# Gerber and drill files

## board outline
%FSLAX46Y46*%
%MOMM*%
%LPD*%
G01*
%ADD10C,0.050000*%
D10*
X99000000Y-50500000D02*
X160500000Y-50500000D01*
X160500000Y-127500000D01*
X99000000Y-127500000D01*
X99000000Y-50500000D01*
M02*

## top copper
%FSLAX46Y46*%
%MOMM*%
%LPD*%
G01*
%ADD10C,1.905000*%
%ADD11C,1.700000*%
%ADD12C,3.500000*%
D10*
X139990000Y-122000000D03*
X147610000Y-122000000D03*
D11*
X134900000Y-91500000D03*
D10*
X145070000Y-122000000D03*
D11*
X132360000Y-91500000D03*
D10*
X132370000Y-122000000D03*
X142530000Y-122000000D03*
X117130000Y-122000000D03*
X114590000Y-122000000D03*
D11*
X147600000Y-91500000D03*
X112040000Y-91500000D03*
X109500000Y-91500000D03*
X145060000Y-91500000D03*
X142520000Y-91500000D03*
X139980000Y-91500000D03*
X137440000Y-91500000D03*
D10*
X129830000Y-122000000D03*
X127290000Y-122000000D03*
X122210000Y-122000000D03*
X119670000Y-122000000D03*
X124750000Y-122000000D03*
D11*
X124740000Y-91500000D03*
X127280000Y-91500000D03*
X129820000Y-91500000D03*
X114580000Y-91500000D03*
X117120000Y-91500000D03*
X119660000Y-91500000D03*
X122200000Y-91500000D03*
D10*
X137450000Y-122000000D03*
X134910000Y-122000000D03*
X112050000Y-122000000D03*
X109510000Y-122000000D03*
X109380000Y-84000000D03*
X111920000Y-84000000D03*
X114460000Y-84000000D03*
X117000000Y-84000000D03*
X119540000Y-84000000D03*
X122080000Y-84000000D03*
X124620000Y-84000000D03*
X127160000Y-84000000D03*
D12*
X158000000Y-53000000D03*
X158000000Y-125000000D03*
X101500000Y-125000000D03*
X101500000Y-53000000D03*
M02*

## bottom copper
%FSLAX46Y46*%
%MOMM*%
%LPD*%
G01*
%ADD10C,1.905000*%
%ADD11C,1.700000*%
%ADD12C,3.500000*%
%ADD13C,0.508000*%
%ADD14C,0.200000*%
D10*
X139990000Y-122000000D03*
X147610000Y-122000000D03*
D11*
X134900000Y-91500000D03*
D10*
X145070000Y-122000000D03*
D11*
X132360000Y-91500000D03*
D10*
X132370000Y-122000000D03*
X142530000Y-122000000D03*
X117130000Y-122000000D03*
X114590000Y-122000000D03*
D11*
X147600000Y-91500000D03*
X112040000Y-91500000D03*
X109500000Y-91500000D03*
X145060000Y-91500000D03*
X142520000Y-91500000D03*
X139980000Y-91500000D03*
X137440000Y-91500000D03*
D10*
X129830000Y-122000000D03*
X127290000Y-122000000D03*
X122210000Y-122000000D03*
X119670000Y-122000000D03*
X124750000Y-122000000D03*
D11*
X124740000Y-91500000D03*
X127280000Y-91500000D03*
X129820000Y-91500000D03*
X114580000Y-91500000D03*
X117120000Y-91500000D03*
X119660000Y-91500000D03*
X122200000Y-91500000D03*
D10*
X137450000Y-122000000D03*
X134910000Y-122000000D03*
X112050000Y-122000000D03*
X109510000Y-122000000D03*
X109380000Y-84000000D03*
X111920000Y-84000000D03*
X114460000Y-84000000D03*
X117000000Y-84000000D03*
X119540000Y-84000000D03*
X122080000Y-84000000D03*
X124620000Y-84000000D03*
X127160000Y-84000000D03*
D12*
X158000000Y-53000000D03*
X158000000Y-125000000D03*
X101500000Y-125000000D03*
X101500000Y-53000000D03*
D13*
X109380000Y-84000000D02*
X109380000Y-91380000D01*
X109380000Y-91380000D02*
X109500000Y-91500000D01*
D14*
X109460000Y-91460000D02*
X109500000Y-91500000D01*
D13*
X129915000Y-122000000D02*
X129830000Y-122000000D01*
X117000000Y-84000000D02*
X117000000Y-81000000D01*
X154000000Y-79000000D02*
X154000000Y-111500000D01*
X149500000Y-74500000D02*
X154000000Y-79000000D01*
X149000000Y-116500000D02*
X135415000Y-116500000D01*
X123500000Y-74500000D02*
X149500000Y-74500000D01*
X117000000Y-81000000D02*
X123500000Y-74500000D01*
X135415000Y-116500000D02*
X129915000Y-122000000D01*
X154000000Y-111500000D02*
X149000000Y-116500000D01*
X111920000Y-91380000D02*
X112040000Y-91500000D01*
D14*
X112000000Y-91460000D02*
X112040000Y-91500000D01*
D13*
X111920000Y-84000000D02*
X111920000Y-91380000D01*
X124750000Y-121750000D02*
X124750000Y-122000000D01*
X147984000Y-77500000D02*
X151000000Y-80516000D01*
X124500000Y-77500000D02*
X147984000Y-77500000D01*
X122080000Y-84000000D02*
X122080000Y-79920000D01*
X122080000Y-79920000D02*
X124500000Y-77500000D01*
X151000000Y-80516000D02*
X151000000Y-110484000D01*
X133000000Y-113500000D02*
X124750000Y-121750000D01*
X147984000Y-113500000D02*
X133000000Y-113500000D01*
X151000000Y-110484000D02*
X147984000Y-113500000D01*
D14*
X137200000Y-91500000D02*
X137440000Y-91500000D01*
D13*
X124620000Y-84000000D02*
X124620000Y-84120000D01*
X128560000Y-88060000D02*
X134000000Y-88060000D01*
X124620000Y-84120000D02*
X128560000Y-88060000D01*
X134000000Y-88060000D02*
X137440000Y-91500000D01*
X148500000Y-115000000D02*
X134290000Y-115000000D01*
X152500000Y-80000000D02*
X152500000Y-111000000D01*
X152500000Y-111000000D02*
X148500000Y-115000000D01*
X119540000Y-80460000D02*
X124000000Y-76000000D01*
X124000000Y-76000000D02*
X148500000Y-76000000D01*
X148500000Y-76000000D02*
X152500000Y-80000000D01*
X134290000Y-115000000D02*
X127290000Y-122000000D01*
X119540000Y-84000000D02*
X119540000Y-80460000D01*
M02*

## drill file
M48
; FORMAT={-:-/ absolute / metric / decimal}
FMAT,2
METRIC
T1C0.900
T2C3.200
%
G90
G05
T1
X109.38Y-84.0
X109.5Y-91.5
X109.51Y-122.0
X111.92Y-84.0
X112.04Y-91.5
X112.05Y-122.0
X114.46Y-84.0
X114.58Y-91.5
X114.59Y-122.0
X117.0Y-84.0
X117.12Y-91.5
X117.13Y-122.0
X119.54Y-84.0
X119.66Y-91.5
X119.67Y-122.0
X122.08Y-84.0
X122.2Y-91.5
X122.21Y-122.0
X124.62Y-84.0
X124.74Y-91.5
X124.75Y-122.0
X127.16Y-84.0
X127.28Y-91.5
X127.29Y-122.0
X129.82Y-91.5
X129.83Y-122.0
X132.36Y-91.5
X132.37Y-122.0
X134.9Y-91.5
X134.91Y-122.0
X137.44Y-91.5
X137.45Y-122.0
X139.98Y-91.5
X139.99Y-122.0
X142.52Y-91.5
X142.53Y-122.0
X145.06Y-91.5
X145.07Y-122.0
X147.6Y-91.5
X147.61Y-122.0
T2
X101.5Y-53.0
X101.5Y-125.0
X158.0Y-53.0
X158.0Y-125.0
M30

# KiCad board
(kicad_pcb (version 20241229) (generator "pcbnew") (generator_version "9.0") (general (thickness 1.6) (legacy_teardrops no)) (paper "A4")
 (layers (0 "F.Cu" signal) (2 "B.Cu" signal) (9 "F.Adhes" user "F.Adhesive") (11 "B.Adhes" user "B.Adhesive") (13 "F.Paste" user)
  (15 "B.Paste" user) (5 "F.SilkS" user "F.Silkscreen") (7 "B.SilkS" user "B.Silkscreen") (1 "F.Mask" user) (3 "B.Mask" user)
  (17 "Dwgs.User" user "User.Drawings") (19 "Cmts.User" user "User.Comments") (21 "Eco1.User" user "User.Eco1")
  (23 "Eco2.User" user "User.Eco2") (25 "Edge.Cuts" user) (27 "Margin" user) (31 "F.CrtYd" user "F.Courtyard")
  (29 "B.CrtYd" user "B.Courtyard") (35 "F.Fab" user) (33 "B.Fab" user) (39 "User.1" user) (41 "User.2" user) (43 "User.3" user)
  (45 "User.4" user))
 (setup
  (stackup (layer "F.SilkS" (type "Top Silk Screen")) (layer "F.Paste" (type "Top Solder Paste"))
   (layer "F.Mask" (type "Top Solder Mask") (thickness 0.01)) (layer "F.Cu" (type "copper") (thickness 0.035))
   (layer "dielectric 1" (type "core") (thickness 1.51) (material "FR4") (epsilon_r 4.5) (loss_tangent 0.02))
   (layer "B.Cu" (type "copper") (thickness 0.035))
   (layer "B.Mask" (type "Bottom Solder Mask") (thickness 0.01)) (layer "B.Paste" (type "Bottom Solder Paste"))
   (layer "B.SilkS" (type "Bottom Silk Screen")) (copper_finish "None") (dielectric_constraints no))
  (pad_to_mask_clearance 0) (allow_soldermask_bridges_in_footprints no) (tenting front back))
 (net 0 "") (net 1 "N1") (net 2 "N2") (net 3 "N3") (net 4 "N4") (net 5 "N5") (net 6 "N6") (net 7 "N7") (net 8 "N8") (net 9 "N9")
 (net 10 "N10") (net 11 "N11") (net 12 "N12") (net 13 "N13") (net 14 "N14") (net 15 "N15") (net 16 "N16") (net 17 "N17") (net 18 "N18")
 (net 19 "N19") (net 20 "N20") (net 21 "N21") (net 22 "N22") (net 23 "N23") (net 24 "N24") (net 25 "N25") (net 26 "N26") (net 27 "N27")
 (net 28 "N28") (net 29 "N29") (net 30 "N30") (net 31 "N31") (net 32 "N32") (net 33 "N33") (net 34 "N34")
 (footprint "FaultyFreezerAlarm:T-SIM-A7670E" (layer "F.Cu") (at 173.81 136.75 90)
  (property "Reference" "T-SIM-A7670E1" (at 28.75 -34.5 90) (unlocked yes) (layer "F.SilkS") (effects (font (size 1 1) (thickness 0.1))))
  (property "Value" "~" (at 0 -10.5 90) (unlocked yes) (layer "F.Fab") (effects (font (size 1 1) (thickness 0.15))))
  (pad "0" thru_hole circle (at 14.75 -33.82) (size 1.905 1.905) (drill 0.9) (layers "*.Cu" "*.Mask") (remove_unused_layers no) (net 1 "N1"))
  (pad "01" thru_hole circle (at 14.75 -26.2) (size 1.905 1.905) (drill 0.9) (layers "*.Cu" "*.Mask") (remove_unused_layers no) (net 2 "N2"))
  (pad "02" thru_hole circle (at 45.25 -38.91) (size 1.7 1.7) (drill 0.9) (layers "*.Cu" "*.Mask") (remove_unused_layers no) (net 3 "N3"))
  (pad "03" thru_hole circle (at 14.75 -28.74) (size 1.905 1.905) (drill 0.9) (layers "*.Cu" "*.Mask") (remove_unused_layers no)
   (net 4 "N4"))
  (pad "04" thru_hole circle (at 45.25 -41.45) (size 1.7 1.7) (drill 0.9) (layers "*.Cu" "*.Mask") (remove_unused_layers no) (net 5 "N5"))
  (pad "05" thru_hole circle (at 14.75 -41.44) (size 1.905 1.905) (drill 0.9) (layers "*.Cu" "*.Mask") (remove_unused_layers no)
   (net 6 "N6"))
  (pad "06" thru_hole circle (at 14.75 -31.28) (size 1.905 1.905) (drill 0.9) (layers "*.Cu" "*.Mask") (remove_unused_layers no)
   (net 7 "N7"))
  (pad "07" thru_hole circle (at 14.75 -56.68) (size 1.905 1.905) (drill 0.9) (layers "*.Cu" "*.Mask") (remove_unused_layers no)
   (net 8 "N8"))
  (pad "08" thru_hole circle (at 14.75 -59.22) (size 1.905 1.905) (drill 0.9) (layers "*.Cu" "*.Mask") (remove_unused_layers no)
   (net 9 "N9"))
  (pad "09" thru_hole circle (at 45.25 -26.21) (size 1.7 1.7) (drill 0.9) (layers "*.Cu" "*.Mask") (remove_unused_layers no) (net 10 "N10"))
  (pad "10" thru_hole circle (at 45.25 -61.77) (size 1.7 1.7) (drill 0.9) (layers "*.Cu" "*.Mask") (remove_unused_layers no) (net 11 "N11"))
  (pad "11" thru_hole circle (at 45.25 -64.31) (size 1.7 1.7) (drill 0.9) (layers "*.Cu" "*.Mask") (remove_unused_layers no) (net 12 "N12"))
  (pad "12" thru_hole circle (at 45.25 -28.75) (size 1.7 1.7) (drill 0.9) (layers "*.Cu" "F.Mask") (remove_unused_layers no) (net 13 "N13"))
  (pad "13" thru_hole circle (at 45.25 -31.29) (size 1.7 1.7) (drill 0.9) (layers "*.Cu" "*.Mask") (remove_unused_layers no) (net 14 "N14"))
  (pad "14" thru_hole circle (at 45.25 -33.83) (size 1.7 1.7) (drill 0.9) (layers "*.Cu" "*.Mask") (remove_unused_layers no) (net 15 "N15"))
  (pad "15" thru_hole circle (at 45.25 -36.37) (size 1.7 1.7) (drill 0.9) (layers "*.Cu" "*.Mask") (remove_unused_layers no) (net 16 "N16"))
  (pad "18" thru_hole circle (at 14.75 -43.98) (size 1.905 1.905) (drill 0.9) (layers "*.Cu" "*.Mask") (remove_unused_layers no)
   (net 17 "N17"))
  (pad "19" thru_hole circle (at 14.75 -46.52) (size 1.905 1.905) (drill 0.9) (layers "*.Cu" "*.Mask") (remove_unused_layers no)
   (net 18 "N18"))
  (pad "21" thru_hole circle (at 14.75 -51.6) (size 1.905 1.905) (drill 0.9) (layers "*.Cu" "*.Mask") (remove_unused_layers no)
   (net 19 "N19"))
  (pad "22" thru_hole circle (at 14.75 -54.14) (size 1.905 1.905) (drill 0.9) (layers "*.Cu" "*.Mask") (remove_unused_layers no)
   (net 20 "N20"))
  (pad "23" thru_hole circle (at 14.75 -49.06) (size 1.905 1.905) (drill 0.9) (layers "*.Cu" "*.Mask") (remove_unused_layers no)
   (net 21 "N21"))
  (pad "25" thru_hole circle (at 45.25 -49.07) (size 1.7 1.7) (drill 0.9) (layers "*.Cu" "*.Mask" "Dwgs.User") (remove_unused_layers no)
   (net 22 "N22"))
  (pad "26" thru_hole circle (at 45.25 -46.53) (size 1.7 1.7) (drill 0.9) (layers "*.Cu" "*.Mask") (remove_unused_layers no) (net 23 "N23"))
  (pad "27" thru_hole circle (at 45.25 -43.99) (size 1.7 1.7) (drill 0.9) (layers "*.Cu" "*.Mask") (remove_unused_layers no) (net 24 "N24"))
  (pad "32" thru_hole circle (at 45.25 -59.23) (size 1.7 1.7) (drill 0.9) (layers "*.Cu" "*.Mask" "Dwgs.User") (remove_unused_layers no)
   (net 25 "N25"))
  (pad "33" thru_hole circle (at 45.25 -56.69) (size 1.7 1.7) (drill 0.9) (layers "*.Cu" "F.Mask") (remove_unused_layers no) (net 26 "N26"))
  (pad "34" thru_hole circle (at 45.25 -54.15) (size 1.7 1.7) (drill 0.9) (layers "*.Cu" "*.Mask") (remove_unused_layers no) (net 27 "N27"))
  (pad "35" thru_hole circle (at 45.25 -51.61) (size 1.7 1.7) (drill 0.9) (layers "*.Cu" "*.Mask") (remove_unused_layers no) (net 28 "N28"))
  (pad "36" thru_hole circle (at 14.75 -36.36) (size 1.905 1.905) (drill 0.9) (layers "*.Cu" "*.Mask") (remove_unused_layers no)
   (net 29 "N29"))
  (pad "39" thru_hole circle (at 14.75 -38.9) (size 1.905 1.905) (drill 0.9) (layers "*.Cu" "F.Mask") (remove_unused_layers no)
   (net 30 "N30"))
  (pad "RX" thru_hole circle (at 14.75 -61.76) (size 1.905 1.905) (drill 0.9) (layers "*.Cu" "*.Mask" "Dwgs.User") (remove_unused_layers no)
   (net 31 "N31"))
  (pad "TX" thru_hole circle (at 14.75 -64.3) (size 1.905 1.905) (drill 0.9) (layers "*.Cu" "*.Mask") (remove_unused_layers no)
   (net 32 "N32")))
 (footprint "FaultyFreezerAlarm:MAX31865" (layer "F.Cu") (at 118.27 84)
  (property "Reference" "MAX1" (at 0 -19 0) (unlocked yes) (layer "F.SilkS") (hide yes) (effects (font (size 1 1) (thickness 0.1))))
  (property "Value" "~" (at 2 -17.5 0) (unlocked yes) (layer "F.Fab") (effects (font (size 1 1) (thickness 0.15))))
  (pad "1" thru_hole circle (at -8.89 0) (size 1.905 1.905) (drill 0.9) (layers "*.Cu" "*.Mask") (remove_unused_layers no) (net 12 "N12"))
  (pad "2" thru_hole circle (at -6.35 0) (size 1.905 1.905) (drill 0.9) (layers "*.Cu" "*.Mask") (remove_unused_layers no) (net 11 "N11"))
  (pad "3" thru_hole circle (at -3.81 0) (size 1.905 1.905) (drill 0.9) (layers "*.Cu" "*.Mask") (remove_unused_layers no) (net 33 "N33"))
  (pad "4" thru_hole circle (at -1.27 0) (size 1.905 1.905) (drill 0.9) (layers "*.Cu" "*.Mask") (remove_unused_layers no) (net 17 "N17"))
  (pad "5" thru_hole circle (at 1.27 0) (size 1.905 1.905) (drill 0.9) (layers "*.Cu" "*.Mask") (remove_unused_layers no) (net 18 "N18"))
  (pad "6" thru_hole circle (at 3.81 0) (size 1.905 1.905) (drill 0.9) (layers "*.Cu" "*.Mask") (remove_unused_layers no) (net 21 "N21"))
  (pad "7" thru_hole circle (at 6.35 0) (size 1.905 1.905) (drill 0.9) (layers "*.Cu" "*.Mask") (remove_unused_layers no) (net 16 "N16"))
  (pad "8" thru_hole circle (at 8.89 0) (size 1.905 1.905) (drill 0.9) (layers "*.Cu" "*.Mask") (remove_unused_layers no) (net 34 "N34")))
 (gr_rect (start 99 50.5) (end 160.5 127.5) (stroke (width 0.05) (type default)) (fill no) (layer "Edge.Cuts"))
 (via (at 158 53) (size 3.5) (drill 3.2) (layers "F.Cu" "B.Cu") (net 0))
 (via (at 158 125) (size 3.5) (drill 3.2) (layers "F.Cu" "B.Cu") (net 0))
 (via (at 101.5 125) (size 3.5) (drill 3.2) (layers "F.Cu" "B.Cu") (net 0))
 (via (at 101.5 53) (size 3.5) (drill 3.2) (layers "F.Cu" "B.Cu") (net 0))
 (segment (start 109.38 84) (end 109.38 91.38) (width 0.508) (layer "B.Cu") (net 12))
 (segment (start 109.38 91.38) (end 109.5 91.5) (width 0.508) (layer "B.Cu") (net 12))
 (segment (start 109.46 91.46) (end 109.5 91.5) (width 0.2) (layer "B.Cu") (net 12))
 (segment (start 129.915 122) (end 129.83 122) (width 0.508) (layer "B.Cu") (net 17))
 (segment (start 117 84) (end 117 81) (width 0.508) (layer "B.Cu") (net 17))
 (segment (start 154 79) (end 154 111.5) (width 0.508) (layer "B.Cu") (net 17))
 (segment (start 149.5 74.5) (end 154 79) (width 0.508) (layer "B.Cu") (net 17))
 (segment (start 149 116.5) (end 135.415 116.5) (width 0.508) (layer "B.Cu") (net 17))
 (segment (start 123.5 74.5) (end 149.5 74.5) (width 0.508) (layer "B.Cu") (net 17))
 (segment (start 117 81) (end 123.5 74.5) (width 0.508) (layer "B.Cu") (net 17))
 (segment (start 135.415 116.5) (end 129.915 122) (width 0.508) (layer "B.Cu") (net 17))
 (segment (start 154 111.5) (end 149 116.5) (width 0.508) (layer "B.Cu") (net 17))
 (segment (start 111.92 91.38) (end 112.04 91.5) (width 0.508) (layer "B.Cu") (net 11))
 (segment (start 112 91.46) (end 112.04 91.5) (width 0.2) (layer "B.Cu") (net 11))
 (segment (start 111.92 84) (end 111.92 91.38) (width 0.508) (layer "B.Cu") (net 11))
 (segment (start 124.75 121.75) (end 124.75 122) (width 0.508) (layer "B.Cu") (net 21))
 (segment (start 147.984 77.5) (end 151 80.516) (width 0.508) (layer "B.Cu") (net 21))
 (segment (start 124.5 77.5) (end 147.984 77.5) (width 0.508) (layer "B.Cu") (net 21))
 (segment (start 122.08 84) (end 122.08 79.92) (width 0.508) (layer "B.Cu") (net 21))
 (segment (start 122.08 79.92) (end 124.5 77.5) (width 0.508) (layer "B.Cu") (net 21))
 (segment (start 151 80.516) (end 151 110.484) (width 0.508) (layer "B.Cu") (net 21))
 (segment (start 133 113.5) (end 124.75 121.75) (width 0.508) (layer "B.Cu") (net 21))
 (segment (start 147.984 113.5) (end 133 113.5) (width 0.508) (layer "B.Cu") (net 21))
 (segment (start 151 110.484) (end 147.984 113.5) (width 0.508) (layer "B.Cu") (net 21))
 (segment (start 137.2 91.5) (end 137.44 91.5) (width 0.2) (layer "B.Cu") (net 16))
 (segment (start 124.62 84) (end 124.62 84.12) (width 0.508) (layer "B.Cu") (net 16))
 (segment (start 128.56 88.06) (end 134 88.06) (width 0.508) (layer "B.Cu") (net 16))
 (segment (start 124.62 84.12) (end 128.56 88.06) (width 0.508) (layer "B.Cu") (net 16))
 (segment (start 134 88.06) (end 137.44 91.5) (width 0.508) (layer "B.Cu") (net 16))
 (segment (start 148.5 115) (end 134.29 115) (width 0.508) (layer "B.Cu") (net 18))
 (segment (start 152.5 80) (end 152.5 111) (width 0.508) (layer "B.Cu") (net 18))
 (segment (start 152.5 111) (end 148.5 115) (width 0.508) (layer "B.Cu") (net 18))
 (segment (start 119.54 80.46) (end 124 76) (width 0.508) (layer "B.Cu") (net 18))
 (segment (start 124 76) (end 148.5 76) (width 0.508) (layer "B.Cu") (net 18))
 (segment (start 148.5 76) (end 152.5 80) (width 0.508) (layer "B.Cu") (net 18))
 (segment (start 134.29 115) (end 127.29 122) (width 0.508) (layer "B.Cu") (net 18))
 (segment (start 119.54 84) (end 119.54 80.46) (width 0.508) (layer "B.Cu") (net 18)))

